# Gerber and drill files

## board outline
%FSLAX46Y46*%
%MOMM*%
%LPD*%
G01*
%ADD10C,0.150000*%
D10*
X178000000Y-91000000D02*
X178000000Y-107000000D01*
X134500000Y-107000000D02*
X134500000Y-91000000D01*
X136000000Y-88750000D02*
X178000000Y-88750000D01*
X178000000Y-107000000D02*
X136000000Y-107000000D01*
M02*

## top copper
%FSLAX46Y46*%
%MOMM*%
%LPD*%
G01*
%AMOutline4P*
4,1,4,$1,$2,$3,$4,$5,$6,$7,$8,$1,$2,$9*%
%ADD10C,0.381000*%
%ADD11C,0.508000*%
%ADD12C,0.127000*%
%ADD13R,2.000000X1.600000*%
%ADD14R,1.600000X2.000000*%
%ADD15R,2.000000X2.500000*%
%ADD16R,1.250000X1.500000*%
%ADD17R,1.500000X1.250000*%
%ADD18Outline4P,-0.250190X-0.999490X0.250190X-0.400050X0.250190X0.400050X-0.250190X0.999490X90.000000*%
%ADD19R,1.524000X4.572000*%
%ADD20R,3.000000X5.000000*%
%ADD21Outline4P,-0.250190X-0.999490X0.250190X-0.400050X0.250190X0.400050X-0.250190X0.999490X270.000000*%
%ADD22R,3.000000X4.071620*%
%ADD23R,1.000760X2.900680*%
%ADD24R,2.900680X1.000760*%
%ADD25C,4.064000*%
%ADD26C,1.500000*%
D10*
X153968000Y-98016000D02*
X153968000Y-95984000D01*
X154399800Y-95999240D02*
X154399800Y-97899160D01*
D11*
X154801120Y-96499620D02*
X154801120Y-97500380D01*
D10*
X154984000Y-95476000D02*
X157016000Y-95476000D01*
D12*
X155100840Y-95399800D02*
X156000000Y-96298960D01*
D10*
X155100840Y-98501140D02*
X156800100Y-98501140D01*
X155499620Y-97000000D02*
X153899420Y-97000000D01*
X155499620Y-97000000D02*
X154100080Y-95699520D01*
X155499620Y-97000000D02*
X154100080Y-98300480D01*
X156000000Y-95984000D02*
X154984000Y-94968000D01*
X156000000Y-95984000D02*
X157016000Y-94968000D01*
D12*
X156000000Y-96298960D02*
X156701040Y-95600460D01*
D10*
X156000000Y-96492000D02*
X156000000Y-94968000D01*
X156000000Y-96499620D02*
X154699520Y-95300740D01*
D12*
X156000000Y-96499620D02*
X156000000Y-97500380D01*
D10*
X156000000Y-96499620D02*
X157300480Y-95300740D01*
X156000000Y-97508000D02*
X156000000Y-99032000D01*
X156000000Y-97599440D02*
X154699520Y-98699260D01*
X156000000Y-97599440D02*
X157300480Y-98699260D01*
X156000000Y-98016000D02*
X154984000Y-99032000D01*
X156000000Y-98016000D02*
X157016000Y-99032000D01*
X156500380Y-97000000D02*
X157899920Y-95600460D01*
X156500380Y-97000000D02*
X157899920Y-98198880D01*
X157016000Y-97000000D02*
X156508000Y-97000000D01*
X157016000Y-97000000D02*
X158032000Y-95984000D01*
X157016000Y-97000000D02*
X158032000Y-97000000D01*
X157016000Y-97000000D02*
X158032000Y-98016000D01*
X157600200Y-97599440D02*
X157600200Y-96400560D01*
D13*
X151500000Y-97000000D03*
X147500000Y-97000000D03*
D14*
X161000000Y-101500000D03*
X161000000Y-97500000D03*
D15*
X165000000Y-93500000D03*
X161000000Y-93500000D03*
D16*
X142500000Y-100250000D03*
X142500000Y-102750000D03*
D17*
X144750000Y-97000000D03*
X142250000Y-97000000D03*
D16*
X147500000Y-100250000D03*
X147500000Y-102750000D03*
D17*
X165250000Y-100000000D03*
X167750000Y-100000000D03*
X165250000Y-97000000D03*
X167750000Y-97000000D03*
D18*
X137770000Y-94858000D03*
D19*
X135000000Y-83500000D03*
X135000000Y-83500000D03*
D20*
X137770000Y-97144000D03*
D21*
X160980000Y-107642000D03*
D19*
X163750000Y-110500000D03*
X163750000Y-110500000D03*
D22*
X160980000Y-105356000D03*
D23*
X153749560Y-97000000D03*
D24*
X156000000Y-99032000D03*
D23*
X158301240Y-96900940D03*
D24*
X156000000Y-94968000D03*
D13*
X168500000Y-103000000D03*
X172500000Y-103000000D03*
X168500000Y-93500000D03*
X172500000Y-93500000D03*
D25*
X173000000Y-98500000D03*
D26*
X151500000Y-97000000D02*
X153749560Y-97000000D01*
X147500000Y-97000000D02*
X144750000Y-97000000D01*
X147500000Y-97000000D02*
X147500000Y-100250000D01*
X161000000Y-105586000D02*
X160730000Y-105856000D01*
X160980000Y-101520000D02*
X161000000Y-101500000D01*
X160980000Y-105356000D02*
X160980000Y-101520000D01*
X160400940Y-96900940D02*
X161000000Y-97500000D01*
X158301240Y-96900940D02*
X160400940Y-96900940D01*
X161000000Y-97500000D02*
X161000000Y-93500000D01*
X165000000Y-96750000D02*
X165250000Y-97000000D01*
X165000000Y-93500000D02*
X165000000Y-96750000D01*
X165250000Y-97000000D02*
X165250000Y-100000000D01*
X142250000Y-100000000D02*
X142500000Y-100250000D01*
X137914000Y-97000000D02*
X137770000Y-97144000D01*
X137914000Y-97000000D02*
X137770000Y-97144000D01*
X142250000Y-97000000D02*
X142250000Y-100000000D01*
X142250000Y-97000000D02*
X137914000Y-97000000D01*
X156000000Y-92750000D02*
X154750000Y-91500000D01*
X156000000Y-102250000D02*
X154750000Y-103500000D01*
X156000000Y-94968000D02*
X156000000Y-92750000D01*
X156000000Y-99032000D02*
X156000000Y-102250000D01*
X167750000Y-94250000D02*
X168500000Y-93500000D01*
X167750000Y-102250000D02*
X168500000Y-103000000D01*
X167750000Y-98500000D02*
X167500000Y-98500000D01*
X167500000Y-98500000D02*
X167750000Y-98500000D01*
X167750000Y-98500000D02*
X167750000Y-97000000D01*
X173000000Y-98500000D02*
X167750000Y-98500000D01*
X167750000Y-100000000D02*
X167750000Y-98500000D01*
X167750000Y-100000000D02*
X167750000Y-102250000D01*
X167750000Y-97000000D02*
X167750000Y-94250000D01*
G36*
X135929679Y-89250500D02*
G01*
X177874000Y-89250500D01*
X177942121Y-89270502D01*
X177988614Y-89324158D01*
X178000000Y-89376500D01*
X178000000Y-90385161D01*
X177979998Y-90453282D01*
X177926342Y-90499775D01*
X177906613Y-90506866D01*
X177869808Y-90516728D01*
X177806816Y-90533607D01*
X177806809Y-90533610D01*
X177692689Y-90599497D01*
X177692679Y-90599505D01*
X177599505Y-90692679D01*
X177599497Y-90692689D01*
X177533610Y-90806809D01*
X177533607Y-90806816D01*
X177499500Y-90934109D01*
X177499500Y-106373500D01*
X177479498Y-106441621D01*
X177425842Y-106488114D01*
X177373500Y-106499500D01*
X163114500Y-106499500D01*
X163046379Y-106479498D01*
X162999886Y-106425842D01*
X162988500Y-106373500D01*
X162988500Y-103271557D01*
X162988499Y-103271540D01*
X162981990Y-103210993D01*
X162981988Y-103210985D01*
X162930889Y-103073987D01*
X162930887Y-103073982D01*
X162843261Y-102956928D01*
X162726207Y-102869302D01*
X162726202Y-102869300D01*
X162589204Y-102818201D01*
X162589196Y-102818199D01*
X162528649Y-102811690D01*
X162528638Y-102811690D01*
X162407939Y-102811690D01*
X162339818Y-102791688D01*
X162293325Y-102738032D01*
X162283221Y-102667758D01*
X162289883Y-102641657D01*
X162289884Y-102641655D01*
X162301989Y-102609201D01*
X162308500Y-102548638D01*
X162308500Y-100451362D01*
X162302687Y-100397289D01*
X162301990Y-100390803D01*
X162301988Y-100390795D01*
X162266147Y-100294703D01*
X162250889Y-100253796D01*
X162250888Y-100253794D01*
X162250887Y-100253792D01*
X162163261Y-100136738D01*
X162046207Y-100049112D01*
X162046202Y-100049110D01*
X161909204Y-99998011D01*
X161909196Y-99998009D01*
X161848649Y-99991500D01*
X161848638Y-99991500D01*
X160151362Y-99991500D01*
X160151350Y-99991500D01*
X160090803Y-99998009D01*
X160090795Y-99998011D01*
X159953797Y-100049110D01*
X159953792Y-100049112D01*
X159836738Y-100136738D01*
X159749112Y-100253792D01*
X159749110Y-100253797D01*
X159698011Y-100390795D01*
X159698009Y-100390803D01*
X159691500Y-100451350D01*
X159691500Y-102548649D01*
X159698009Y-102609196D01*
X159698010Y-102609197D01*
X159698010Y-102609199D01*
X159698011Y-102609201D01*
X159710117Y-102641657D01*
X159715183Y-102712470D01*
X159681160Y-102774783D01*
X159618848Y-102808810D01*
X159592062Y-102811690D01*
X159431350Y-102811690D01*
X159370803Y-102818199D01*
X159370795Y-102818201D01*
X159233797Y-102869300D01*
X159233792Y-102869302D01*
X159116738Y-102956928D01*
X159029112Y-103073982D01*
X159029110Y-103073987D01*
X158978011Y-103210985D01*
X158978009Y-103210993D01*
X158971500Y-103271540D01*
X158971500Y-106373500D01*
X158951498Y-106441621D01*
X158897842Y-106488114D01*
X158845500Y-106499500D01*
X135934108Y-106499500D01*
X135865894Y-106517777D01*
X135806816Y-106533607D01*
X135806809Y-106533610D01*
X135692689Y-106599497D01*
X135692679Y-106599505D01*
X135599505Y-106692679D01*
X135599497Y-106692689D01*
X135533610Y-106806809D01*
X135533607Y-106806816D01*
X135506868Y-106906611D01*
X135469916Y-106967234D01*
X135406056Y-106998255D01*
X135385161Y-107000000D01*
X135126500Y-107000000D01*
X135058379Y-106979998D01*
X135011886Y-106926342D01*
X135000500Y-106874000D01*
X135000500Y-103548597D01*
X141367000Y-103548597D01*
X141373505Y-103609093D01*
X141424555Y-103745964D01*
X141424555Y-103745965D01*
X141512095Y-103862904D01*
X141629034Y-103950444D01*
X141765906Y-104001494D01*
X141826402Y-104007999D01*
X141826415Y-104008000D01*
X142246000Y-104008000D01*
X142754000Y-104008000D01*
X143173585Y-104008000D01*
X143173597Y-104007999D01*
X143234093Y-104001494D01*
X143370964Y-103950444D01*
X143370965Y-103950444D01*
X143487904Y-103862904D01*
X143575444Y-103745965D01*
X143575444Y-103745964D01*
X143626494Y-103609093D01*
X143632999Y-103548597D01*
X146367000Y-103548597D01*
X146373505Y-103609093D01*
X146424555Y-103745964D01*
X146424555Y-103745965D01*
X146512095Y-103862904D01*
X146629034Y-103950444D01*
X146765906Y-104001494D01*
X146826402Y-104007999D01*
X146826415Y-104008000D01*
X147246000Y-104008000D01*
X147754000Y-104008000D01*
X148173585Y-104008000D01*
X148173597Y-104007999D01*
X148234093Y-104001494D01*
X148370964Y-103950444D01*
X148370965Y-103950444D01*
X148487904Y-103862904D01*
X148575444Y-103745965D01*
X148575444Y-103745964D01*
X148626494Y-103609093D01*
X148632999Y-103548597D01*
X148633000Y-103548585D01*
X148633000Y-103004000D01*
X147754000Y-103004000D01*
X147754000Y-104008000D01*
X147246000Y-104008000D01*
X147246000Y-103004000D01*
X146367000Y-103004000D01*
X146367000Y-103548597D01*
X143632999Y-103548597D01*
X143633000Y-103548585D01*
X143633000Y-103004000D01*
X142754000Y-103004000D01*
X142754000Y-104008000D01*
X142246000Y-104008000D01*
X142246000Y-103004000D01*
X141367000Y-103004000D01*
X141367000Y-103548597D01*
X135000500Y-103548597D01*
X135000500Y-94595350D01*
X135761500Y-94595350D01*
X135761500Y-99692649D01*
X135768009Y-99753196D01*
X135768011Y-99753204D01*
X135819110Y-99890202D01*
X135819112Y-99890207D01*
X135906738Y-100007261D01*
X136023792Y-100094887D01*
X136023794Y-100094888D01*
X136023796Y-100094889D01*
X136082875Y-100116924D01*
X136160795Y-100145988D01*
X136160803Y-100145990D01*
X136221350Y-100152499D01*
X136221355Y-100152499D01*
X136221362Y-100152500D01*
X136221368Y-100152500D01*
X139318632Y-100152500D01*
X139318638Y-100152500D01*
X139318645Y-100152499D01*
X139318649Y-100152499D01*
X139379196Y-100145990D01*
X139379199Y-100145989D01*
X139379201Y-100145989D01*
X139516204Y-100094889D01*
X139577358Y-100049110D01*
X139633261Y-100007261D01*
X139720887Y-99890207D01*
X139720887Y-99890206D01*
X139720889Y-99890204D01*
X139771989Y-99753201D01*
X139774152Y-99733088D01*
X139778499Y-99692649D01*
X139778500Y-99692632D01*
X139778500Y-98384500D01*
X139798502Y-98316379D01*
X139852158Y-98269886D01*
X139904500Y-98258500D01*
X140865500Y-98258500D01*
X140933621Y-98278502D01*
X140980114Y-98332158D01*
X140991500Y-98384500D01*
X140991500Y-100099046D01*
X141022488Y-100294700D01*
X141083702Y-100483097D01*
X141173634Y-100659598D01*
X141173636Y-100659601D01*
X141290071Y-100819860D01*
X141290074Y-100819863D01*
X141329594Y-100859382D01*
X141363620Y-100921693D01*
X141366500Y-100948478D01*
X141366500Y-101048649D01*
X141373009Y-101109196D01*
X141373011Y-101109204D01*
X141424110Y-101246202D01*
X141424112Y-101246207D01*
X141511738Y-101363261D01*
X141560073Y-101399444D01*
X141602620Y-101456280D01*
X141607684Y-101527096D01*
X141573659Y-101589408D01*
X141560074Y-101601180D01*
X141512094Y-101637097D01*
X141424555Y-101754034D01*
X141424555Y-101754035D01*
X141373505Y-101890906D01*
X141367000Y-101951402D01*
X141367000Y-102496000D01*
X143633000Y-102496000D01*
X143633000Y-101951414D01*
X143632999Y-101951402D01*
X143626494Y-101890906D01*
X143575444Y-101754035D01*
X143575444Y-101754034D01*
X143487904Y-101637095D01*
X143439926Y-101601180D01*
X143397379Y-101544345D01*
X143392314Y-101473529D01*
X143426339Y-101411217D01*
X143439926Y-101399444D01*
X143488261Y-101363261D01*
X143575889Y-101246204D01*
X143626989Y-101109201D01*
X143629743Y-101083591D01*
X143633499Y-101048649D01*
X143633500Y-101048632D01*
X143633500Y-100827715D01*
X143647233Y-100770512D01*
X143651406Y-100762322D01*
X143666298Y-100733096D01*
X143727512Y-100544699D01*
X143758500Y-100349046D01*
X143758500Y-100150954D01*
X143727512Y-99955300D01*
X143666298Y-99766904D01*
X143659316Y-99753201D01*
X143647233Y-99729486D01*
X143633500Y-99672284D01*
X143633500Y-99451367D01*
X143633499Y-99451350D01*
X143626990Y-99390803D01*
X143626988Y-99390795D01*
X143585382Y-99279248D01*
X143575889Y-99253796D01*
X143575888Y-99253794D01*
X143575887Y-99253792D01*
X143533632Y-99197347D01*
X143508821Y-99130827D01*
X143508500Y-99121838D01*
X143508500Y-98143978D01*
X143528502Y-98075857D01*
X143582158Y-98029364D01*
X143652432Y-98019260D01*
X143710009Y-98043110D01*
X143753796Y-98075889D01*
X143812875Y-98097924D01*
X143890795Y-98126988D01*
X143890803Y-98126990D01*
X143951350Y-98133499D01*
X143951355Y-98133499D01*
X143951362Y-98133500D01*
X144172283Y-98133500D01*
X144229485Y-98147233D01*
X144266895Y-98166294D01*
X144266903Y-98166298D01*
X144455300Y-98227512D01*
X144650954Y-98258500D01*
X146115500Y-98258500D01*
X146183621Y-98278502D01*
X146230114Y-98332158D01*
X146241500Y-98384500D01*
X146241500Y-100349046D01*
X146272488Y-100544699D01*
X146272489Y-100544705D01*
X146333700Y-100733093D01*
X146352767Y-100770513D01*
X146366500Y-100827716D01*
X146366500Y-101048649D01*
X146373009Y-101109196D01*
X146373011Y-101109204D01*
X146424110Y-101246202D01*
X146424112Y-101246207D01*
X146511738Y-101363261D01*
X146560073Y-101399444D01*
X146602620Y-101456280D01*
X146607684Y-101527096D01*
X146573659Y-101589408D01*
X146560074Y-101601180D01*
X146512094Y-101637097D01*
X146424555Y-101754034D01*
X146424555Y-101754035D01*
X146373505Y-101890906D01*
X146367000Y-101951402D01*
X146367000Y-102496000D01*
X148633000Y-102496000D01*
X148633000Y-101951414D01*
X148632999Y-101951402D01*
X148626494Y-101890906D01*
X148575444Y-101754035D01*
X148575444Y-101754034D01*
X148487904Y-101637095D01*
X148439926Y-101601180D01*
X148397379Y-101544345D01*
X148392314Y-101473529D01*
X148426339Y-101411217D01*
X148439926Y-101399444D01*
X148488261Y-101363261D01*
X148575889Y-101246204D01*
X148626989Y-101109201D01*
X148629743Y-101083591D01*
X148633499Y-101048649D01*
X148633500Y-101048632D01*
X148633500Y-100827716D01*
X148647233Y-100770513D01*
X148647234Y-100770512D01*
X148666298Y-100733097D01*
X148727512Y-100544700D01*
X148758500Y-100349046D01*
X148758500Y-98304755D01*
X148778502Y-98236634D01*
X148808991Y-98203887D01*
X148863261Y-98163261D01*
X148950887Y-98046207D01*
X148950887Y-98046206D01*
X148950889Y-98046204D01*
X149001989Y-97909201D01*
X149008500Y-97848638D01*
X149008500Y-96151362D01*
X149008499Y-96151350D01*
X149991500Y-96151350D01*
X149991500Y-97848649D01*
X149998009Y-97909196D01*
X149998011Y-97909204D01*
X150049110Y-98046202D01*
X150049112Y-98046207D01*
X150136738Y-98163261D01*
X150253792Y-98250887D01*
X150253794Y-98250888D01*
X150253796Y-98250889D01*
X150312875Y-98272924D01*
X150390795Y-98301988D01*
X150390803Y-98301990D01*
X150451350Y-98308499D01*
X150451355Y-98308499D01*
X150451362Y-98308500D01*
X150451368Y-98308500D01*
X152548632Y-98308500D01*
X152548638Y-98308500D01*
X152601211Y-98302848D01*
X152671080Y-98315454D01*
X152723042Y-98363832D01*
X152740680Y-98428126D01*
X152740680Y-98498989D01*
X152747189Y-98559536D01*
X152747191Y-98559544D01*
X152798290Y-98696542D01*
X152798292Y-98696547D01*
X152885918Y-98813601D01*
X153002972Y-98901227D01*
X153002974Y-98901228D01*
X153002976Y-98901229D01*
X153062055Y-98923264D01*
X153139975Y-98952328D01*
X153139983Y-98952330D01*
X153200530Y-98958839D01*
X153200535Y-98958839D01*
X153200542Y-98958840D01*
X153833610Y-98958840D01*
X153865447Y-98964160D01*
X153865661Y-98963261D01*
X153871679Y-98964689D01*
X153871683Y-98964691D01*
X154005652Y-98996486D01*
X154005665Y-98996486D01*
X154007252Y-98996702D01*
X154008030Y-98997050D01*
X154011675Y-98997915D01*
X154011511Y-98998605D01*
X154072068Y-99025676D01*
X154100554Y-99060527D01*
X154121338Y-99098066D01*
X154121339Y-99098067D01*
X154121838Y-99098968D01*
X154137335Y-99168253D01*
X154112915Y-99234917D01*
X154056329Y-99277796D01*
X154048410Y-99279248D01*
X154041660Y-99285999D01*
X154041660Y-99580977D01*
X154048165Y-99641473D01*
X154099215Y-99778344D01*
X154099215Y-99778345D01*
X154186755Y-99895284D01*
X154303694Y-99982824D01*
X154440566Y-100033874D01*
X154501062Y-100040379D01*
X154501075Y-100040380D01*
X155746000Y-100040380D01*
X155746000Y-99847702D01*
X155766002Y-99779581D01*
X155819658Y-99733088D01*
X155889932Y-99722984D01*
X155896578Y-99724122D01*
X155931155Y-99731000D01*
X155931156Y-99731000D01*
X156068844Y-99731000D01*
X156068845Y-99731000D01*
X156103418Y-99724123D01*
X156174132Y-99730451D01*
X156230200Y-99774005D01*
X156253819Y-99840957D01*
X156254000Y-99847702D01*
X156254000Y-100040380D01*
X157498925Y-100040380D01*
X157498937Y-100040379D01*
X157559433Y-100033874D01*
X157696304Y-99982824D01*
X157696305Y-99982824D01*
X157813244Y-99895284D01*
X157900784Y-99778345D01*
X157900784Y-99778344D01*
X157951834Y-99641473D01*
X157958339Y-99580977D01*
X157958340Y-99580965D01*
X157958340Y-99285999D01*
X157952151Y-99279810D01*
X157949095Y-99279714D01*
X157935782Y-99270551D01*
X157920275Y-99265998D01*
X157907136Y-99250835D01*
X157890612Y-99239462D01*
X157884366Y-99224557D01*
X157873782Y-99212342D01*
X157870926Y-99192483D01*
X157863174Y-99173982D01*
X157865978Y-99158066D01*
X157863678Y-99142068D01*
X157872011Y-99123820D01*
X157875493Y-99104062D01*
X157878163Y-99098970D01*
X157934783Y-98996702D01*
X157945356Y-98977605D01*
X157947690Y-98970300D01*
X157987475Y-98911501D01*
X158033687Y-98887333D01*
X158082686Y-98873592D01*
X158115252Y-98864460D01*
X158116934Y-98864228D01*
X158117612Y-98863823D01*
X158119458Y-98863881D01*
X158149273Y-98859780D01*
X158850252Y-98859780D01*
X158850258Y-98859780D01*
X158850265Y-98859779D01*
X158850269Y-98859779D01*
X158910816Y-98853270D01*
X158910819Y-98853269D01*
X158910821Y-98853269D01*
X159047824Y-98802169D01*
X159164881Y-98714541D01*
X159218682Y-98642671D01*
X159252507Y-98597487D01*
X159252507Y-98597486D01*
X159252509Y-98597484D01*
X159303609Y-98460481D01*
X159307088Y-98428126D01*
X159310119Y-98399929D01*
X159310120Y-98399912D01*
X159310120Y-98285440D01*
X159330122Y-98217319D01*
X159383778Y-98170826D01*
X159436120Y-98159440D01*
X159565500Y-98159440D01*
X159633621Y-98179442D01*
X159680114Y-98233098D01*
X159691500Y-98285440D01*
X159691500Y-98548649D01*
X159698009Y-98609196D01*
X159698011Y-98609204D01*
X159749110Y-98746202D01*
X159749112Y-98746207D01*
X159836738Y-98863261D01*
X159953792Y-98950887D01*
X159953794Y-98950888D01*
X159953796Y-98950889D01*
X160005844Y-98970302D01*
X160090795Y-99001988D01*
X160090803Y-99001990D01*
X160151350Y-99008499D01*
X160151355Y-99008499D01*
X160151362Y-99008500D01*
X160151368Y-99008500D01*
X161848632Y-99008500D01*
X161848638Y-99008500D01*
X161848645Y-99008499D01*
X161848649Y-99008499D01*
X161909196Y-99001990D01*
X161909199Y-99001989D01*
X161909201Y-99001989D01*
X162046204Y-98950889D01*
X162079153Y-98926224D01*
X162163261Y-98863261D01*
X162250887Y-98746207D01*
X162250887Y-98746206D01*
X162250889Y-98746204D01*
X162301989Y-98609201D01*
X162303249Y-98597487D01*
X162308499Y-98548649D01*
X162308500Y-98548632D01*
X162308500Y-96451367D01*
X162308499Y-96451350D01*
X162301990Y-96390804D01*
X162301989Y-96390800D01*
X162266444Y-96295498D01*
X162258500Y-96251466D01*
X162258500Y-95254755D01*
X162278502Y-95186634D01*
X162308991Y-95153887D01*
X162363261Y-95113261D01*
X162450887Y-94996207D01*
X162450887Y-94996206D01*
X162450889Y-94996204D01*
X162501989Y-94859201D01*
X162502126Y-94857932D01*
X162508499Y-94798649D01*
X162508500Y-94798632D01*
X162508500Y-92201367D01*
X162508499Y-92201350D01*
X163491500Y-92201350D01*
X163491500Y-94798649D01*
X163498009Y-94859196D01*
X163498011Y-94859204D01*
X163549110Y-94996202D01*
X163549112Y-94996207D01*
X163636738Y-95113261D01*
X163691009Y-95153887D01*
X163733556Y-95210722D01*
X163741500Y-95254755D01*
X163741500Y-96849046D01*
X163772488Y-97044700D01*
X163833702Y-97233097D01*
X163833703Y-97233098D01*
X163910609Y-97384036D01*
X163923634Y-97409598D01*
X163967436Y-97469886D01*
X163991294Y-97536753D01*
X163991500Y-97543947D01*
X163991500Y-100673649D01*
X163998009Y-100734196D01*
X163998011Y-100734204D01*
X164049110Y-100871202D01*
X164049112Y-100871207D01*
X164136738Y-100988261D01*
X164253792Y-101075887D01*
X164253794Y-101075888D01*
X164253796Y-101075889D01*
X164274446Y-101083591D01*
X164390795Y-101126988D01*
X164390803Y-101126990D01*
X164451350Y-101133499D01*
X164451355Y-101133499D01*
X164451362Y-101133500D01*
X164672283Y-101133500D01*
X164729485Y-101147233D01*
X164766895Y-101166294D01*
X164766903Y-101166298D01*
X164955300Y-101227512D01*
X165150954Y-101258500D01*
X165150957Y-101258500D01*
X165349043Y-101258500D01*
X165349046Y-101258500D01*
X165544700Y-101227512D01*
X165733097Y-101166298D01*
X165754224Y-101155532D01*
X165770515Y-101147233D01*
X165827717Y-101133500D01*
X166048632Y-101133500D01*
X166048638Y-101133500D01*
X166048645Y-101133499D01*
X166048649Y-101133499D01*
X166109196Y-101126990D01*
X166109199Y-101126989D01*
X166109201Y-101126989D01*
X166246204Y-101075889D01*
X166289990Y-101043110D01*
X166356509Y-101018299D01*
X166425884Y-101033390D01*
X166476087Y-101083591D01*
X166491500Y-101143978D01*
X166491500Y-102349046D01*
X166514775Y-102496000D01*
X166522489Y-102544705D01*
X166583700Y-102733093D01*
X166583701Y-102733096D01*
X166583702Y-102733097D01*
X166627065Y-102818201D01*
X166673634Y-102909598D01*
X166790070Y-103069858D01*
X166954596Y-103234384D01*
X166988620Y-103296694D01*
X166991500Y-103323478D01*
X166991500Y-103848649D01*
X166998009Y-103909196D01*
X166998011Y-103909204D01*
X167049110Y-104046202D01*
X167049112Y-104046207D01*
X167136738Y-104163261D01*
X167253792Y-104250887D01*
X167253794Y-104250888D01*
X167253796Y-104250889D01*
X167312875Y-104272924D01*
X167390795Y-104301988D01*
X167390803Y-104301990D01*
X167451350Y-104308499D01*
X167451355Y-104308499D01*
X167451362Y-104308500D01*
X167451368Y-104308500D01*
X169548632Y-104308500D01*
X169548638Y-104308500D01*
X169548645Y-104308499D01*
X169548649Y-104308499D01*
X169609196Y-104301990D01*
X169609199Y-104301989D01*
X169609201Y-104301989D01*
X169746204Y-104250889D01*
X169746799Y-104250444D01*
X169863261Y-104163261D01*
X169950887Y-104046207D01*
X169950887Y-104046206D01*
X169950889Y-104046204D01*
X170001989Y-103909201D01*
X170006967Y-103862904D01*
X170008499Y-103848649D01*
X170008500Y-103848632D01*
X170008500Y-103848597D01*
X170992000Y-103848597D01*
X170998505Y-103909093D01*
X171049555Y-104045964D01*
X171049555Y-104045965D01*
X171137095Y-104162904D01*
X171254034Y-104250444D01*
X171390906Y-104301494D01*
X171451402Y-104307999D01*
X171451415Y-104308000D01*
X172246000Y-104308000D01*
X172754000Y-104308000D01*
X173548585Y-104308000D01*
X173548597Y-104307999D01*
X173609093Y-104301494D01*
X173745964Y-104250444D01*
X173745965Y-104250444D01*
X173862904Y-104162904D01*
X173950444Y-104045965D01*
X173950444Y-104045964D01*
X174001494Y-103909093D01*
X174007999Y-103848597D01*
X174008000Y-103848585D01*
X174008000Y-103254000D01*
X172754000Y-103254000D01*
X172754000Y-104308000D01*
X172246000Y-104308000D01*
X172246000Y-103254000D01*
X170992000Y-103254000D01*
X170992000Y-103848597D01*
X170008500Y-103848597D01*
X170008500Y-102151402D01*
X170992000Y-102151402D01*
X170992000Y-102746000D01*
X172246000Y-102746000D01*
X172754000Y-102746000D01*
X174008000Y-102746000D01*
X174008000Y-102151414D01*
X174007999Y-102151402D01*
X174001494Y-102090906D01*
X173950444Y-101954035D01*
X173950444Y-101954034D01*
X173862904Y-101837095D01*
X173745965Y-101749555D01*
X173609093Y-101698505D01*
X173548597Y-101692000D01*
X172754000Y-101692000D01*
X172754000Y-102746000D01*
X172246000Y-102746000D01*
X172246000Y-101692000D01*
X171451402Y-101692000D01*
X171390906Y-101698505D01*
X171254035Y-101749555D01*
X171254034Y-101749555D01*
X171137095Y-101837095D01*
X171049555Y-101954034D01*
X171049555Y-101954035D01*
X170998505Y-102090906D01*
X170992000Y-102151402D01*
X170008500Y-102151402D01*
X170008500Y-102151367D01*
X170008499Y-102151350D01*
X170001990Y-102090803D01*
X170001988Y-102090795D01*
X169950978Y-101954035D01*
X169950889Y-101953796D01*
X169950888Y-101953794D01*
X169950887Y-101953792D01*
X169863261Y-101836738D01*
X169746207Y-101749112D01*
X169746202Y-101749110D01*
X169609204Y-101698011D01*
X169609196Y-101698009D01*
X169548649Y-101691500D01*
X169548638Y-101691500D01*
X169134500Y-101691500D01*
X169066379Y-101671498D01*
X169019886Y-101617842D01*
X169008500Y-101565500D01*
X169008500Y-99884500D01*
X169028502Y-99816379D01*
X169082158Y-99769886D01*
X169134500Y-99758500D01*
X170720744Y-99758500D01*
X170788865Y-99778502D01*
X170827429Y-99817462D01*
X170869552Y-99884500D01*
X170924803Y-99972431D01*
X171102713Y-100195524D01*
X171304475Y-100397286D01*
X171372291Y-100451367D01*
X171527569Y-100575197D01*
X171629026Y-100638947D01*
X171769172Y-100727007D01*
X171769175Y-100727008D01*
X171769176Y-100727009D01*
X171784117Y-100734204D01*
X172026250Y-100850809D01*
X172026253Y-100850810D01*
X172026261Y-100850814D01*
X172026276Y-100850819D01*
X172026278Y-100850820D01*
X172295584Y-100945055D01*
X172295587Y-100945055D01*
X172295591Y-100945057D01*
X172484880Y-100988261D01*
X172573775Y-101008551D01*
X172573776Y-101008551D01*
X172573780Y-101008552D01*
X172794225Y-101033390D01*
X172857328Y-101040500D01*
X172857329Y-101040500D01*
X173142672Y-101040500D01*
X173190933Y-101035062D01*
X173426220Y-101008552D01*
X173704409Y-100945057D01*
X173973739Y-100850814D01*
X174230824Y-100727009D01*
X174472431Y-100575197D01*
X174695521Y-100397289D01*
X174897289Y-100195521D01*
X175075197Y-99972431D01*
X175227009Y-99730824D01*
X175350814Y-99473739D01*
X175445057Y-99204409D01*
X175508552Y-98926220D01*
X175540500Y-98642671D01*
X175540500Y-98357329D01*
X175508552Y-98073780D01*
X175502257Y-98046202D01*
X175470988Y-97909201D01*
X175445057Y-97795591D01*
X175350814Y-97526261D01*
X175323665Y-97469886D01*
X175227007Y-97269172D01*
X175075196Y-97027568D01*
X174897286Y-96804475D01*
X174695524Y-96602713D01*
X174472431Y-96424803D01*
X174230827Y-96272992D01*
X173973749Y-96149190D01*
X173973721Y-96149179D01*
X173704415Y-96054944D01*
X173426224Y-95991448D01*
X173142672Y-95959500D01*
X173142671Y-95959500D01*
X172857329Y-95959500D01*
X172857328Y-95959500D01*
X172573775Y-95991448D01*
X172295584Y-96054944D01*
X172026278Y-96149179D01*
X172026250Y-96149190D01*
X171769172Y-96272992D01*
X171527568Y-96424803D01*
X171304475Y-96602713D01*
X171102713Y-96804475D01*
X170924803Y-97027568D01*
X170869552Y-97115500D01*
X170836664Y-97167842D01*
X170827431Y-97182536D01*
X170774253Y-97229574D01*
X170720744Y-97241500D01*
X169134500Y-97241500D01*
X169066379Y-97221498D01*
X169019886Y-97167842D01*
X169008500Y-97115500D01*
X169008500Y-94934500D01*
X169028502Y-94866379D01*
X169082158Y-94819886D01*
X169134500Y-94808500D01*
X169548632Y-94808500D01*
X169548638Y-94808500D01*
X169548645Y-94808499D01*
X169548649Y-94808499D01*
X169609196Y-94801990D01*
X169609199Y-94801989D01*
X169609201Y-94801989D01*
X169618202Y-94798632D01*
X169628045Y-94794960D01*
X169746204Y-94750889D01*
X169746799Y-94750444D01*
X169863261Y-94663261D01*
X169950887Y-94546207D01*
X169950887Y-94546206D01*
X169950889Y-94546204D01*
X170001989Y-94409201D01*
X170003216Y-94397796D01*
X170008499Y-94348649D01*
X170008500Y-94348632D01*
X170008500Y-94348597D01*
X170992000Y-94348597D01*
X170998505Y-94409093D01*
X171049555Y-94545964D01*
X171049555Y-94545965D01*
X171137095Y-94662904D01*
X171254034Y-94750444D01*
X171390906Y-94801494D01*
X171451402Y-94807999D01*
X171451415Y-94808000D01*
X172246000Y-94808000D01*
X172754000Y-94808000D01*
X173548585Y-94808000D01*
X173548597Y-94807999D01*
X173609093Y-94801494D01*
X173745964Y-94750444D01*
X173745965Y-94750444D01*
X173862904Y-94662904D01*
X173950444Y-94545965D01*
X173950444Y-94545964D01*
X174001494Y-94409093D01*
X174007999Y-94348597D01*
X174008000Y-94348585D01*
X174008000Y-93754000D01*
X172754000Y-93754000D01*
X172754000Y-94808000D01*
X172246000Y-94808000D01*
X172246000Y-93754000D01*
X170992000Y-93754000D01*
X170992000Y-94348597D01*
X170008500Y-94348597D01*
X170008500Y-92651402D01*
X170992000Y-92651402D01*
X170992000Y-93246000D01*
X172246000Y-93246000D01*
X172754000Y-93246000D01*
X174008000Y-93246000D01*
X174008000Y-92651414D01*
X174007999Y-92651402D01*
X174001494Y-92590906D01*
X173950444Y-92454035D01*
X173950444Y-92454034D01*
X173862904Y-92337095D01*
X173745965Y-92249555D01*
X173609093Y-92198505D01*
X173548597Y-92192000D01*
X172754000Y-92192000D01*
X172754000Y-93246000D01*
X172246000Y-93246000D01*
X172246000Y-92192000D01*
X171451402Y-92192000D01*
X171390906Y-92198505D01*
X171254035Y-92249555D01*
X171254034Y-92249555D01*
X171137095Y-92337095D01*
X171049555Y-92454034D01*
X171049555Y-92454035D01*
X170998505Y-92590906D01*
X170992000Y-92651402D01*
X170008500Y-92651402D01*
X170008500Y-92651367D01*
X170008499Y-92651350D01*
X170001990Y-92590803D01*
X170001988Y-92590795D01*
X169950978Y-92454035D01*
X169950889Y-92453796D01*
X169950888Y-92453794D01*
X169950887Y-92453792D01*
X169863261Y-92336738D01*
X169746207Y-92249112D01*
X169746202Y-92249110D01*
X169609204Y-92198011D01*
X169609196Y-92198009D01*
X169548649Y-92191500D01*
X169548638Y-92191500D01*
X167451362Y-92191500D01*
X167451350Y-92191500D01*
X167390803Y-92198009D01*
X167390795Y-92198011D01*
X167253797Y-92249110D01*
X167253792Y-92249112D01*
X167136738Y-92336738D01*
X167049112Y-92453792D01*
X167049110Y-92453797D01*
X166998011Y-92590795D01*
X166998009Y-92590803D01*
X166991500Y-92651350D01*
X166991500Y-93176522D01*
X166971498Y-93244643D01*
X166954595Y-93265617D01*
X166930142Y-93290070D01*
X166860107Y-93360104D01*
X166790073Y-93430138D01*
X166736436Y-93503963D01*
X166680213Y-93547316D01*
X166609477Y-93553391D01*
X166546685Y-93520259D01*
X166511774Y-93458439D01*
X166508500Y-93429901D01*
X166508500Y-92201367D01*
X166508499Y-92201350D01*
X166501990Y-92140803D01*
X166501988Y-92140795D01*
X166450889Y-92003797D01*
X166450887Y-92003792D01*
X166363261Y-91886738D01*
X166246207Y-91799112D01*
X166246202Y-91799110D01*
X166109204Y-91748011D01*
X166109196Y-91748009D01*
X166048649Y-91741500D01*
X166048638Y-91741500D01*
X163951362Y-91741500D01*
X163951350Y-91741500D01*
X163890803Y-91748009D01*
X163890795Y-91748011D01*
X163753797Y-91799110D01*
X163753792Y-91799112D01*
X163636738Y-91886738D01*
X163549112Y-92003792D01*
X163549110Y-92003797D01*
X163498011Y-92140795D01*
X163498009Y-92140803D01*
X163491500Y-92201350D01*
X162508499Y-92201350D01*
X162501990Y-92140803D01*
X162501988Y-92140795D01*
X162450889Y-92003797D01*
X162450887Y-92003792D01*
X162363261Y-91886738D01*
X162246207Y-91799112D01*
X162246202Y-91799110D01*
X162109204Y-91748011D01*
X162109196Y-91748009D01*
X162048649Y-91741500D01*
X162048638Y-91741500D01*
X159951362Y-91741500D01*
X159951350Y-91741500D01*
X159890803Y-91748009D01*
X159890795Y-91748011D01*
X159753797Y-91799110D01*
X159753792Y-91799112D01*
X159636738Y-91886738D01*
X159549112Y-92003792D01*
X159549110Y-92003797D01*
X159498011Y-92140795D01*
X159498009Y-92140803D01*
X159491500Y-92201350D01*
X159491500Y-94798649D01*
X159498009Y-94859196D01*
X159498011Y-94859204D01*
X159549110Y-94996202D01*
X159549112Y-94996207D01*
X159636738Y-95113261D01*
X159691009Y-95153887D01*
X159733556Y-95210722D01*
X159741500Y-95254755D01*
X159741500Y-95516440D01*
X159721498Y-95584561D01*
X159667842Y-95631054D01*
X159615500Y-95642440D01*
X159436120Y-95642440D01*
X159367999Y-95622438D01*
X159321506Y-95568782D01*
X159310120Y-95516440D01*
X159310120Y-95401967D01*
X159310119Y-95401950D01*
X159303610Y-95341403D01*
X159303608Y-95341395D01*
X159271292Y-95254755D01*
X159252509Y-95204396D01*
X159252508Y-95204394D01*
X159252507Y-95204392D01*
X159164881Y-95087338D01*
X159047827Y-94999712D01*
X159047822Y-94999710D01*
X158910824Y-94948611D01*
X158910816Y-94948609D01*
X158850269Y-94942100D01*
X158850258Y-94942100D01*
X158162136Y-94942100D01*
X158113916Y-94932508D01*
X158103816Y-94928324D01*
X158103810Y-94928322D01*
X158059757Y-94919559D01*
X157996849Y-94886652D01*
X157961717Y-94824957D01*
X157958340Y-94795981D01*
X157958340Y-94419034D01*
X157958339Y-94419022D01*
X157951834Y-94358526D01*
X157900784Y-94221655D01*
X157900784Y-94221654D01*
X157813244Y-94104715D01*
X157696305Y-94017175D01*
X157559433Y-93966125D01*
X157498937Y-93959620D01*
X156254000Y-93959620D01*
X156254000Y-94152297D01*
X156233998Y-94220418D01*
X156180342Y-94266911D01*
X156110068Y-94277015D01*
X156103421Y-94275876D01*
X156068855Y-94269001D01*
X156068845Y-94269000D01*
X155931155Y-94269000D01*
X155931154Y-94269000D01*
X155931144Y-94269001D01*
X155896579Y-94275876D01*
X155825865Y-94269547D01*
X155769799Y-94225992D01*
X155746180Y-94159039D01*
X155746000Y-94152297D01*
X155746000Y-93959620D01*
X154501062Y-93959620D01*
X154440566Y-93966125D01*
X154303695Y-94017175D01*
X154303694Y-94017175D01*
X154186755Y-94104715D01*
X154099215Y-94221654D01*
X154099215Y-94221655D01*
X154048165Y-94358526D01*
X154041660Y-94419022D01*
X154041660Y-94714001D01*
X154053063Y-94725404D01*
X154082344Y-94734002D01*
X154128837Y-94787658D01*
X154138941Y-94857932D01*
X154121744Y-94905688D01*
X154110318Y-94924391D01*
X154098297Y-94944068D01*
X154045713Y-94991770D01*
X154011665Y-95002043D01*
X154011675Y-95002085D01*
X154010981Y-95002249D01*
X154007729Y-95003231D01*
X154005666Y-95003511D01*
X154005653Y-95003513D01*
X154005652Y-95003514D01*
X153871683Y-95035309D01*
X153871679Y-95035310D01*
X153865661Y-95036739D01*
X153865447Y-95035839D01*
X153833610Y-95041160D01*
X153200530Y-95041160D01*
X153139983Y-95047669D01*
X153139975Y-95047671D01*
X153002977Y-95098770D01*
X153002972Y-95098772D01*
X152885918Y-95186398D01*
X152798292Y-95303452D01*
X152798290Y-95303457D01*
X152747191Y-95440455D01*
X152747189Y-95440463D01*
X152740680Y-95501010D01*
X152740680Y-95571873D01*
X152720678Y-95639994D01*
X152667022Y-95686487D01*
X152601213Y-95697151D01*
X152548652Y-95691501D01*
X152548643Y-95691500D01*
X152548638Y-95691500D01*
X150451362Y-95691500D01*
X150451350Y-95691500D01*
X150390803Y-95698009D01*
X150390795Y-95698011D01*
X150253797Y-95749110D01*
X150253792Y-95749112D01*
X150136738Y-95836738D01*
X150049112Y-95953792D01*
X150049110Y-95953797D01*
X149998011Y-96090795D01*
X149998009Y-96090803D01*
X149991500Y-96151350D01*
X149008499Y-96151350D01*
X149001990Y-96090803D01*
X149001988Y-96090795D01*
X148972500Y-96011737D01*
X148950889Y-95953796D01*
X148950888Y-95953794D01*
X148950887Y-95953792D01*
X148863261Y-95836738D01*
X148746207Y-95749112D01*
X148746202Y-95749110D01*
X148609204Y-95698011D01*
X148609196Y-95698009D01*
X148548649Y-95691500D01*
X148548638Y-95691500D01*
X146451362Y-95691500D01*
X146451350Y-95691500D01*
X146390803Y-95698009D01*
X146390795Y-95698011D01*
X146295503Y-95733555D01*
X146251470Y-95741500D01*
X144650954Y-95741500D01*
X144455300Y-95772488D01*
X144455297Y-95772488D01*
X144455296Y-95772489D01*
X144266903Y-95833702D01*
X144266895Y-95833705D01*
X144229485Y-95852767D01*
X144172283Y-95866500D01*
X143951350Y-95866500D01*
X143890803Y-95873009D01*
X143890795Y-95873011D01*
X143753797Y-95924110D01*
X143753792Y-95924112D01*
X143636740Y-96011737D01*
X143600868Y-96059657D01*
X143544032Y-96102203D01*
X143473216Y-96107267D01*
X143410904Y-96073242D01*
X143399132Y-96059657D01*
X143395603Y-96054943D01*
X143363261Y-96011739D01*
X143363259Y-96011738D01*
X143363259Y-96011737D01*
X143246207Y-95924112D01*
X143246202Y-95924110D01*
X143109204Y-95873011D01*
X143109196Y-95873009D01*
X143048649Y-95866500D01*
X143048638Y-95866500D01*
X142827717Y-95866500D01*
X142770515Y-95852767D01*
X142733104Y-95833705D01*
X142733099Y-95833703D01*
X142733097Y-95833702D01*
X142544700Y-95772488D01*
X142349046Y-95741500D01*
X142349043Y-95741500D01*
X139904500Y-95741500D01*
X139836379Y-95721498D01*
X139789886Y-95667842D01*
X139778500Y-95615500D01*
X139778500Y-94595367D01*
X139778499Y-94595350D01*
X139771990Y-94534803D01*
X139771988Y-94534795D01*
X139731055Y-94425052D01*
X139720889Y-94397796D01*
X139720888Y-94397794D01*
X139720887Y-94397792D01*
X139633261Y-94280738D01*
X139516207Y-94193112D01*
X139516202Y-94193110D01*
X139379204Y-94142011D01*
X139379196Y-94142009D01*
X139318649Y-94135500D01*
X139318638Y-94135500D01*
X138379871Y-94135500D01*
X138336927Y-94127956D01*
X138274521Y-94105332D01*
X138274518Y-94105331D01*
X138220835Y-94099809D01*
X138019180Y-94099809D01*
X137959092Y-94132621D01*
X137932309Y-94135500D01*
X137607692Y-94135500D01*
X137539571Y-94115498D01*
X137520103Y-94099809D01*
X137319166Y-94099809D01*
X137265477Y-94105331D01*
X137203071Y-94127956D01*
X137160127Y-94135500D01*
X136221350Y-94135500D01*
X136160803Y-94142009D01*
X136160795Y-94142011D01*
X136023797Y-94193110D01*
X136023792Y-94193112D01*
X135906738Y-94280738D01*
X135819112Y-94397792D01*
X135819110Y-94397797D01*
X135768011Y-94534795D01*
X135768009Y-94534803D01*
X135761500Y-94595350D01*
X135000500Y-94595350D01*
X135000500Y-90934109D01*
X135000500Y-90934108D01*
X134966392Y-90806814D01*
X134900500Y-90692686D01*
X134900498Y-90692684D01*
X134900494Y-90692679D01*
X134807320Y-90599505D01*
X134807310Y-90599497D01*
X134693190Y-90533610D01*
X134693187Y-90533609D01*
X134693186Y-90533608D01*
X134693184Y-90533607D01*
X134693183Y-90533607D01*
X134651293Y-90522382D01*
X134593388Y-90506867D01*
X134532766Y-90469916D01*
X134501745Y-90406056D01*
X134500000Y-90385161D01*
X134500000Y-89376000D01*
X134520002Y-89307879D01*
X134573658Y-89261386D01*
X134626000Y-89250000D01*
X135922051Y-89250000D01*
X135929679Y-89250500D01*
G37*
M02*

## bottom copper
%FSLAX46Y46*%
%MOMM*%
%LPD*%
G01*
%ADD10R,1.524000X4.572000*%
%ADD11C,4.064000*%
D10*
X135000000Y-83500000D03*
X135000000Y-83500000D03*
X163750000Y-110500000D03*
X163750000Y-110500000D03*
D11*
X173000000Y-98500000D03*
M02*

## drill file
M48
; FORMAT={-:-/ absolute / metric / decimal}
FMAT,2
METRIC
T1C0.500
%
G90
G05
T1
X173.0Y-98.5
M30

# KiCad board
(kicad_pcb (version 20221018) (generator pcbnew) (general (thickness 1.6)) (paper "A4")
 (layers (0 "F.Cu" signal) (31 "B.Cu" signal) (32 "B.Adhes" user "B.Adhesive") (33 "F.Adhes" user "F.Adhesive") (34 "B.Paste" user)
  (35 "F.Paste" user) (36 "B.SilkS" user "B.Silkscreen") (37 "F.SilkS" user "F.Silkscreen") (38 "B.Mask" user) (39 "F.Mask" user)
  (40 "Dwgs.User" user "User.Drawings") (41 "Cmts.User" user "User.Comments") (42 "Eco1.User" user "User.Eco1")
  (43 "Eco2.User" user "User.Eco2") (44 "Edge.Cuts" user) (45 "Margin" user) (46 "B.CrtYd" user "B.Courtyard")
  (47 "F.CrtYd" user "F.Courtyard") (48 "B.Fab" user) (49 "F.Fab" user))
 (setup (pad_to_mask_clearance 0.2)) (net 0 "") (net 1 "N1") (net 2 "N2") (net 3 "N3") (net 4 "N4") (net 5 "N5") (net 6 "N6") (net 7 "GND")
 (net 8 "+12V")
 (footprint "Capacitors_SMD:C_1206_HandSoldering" (layer "F.Cu") (at 149.5 97 180)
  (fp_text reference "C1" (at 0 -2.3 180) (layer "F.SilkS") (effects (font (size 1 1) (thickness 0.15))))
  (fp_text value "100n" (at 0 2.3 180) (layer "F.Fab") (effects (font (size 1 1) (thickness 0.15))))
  (pad "1" smd rect (at -2 0 180) (size 2 1.6) (layers "F.Cu" "F.Paste" "F.Mask") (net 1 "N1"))
  (pad "2" smd rect (at 2 0 180) (size 2 1.6) (layers "F.Cu" "F.Paste" "F.Mask") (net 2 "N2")))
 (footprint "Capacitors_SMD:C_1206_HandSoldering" (layer "F.Cu") (at 161 99.5 90)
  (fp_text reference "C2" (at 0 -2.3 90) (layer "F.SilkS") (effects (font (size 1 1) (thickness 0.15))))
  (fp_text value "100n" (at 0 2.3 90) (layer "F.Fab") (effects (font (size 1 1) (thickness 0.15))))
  (pad "1" smd rect (at -2 0 90) (size 2 1.6) (layers "F.Cu" "F.Paste" "F.Mask") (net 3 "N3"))
  (pad "2" smd rect (at 2 0 90) (size 2 1.6) (layers "F.Cu" "F.Paste" "F.Mask") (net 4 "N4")))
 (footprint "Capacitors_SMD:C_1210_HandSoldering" (layer "F.Cu") (at 163 93.5 180)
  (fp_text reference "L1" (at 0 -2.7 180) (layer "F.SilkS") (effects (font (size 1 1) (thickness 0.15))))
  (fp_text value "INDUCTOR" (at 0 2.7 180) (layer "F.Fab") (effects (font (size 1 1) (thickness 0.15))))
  (pad "1" smd rect (at -2 0 180) (size 2 2.5) (layers "F.Cu" "F.Paste" "F.Mask") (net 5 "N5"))
  (pad "2" smd rect (at 2 0 180) (size 2 2.5) (layers "F.Cu" "F.Paste" "F.Mask") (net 4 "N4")))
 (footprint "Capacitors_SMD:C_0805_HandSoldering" (layer "F.Cu") (at 142.5 101.5 -90)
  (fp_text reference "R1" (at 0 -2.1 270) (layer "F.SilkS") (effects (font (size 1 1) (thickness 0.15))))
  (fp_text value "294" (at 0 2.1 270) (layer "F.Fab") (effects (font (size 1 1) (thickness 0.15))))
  (pad "1" smd rect (at -1.25 0 270) (size 1.5 1.25) (layers "F.Cu" "F.Paste" "F.Mask") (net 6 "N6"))
  (pad "2" smd rect (at 1.25 0 270) (size 1.5 1.25) (layers "F.Cu" "F.Paste" "F.Mask") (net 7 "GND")))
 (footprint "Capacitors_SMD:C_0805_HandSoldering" (layer "F.Cu") (at 143.5 97 180)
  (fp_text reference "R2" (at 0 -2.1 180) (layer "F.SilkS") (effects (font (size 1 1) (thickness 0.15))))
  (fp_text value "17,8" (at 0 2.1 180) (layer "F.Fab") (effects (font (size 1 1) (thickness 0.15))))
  (pad "1" smd rect (at -1.25 0 180) (size 1.5 1.25) (layers "F.Cu" "F.Paste" "F.Mask") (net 2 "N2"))
  (pad "2" smd rect (at 1.25 0 180) (size 1.5 1.25) (layers "F.Cu" "F.Paste" "F.Mask") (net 6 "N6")))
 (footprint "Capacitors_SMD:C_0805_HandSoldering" (layer "F.Cu") (at 147.5 101.5 -90)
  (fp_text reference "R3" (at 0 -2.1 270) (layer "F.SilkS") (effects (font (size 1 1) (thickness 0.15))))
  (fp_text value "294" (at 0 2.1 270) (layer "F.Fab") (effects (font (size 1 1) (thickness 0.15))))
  (pad "1" smd rect (at -1.25 0 270) (size 1.5 1.25) (layers "F.Cu" "F.Paste" "F.Mask") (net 2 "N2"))
  (pad "2" smd rect (at 1.25 0 270) (size 1.5 1.25) (layers "F.Cu" "F.Paste" "F.Mask") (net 7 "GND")))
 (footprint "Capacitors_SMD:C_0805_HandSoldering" (layer "F.Cu") (at 166.5 100)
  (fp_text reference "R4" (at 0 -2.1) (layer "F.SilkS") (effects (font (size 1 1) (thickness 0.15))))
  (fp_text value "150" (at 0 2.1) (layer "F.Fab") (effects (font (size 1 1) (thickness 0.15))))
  (pad "1" smd rect (at -1.25 0) (size 1.5 1.25) (layers "F.Cu" "F.Paste" "F.Mask") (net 5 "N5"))
  (pad "2" smd rect (at 1.25 0) (size 1.5 1.25) (layers "F.Cu" "F.Paste" "F.Mask") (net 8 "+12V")))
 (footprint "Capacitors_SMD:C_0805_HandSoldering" (layer "F.Cu") (at 166.5 97)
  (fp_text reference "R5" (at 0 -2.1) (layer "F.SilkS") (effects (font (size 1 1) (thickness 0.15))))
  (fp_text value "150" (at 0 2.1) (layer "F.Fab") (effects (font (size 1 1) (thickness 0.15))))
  (pad "1" smd rect (at -1.25 0) (size 1.5 1.25) (layers "F.Cu" "F.Paste" "F.Mask") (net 5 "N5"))
  (pad "2" smd rect (at 1.25 0) (size 1.5 1.25) (layers "F.Cu" "F.Paste" "F.Mask") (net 8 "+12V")))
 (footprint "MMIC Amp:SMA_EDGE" (layer "F.Cu") (at 136.5 88 90)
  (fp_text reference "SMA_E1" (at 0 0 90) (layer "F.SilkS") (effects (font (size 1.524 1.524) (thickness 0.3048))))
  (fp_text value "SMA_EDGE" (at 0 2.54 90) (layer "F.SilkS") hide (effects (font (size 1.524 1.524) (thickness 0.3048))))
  (pad "1" connect trapezoid (at -6.858 1.27 90) (size 0.50038 1.39954) (rect_delta 0.59944 0) (layers "F.Cu" "F.Mask") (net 7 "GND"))
  (pad "1" connect rect (at 4.5 -1.5 90) (size 4.572 1.524) (layers "*.Cu" "F.Mask") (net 7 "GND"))
  (pad "2" connect rect (at 4.5 -1.5 90) (size 4.572 1.524) (layers "*.Cu" "F.Mask") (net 7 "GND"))
  (pad "3" connect rect (at -9.144 1.27 90) (size 5 3) (layers "F.Cu" "F.Mask") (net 6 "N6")))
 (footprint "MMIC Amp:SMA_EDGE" (layer "F.Cu") (at 162.25 114.5 -90)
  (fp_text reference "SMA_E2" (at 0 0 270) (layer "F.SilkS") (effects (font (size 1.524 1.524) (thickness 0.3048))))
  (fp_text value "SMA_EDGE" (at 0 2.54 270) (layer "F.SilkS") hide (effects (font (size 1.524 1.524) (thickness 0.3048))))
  (pad "1" connect trapezoid (at -6.858 1.27 270) (size 0.50038 1.39954) (rect_delta 0.59944 0) (layers "F.Cu" "F.Mask") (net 7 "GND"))
  (pad "1" connect rect (at -4 -1.5 270) (size 4.572 1.524) (layers "*.Cu" "F.Mask") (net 7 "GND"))
  (pad "2" connect rect (at -4 -1.5 270) (size 4.572 1.524) (layers "*.Cu" "F.Mask") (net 7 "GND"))
  (pad "3" connect rect (at -9.144 1.27 270) (size 4.07162 3) (layers "F.Cu" "F.Mask") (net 3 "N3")))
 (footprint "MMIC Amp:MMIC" (layer "F.Cu") (at 156 97)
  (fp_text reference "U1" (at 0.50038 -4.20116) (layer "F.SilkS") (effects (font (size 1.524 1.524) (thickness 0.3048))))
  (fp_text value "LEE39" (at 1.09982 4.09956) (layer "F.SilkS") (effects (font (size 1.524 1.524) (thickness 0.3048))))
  (fp_line (start -2.032 1.016) (end -2.032 -1.016) (stroke (width 0.381) (type solid)) (layer "F.Cu"))
  (fp_line (start -1.6002 -1.00076) (end -1.6002 0.89916) (stroke (width 0.381) (type solid)) (layer "F.Cu"))
  (fp_line (start -1.19888 -0.50038) (end -1.19888 0.50038) (stroke (width 0.508) (type solid)) (layer "F.Cu"))
  (fp_line (start -1.016 -1.524) (end 1.016 -1.524) (stroke (width 0.381) (type solid)) (layer "F.Cu"))
  (fp_line (start -0.89916 -1.6002) (end 0 -0.70104) (stroke (width 0.127) (type solid)) (layer "F.Cu"))
  (fp_line (start -0.89916 1.50114) (end 0.8001 1.50114) (stroke (width 0.381) (type solid)) (layer "F.Cu"))
  (fp_line (start -0.50038 0) (end -2.10058 0) (stroke (width 0.381) (type solid)) (layer "F.Cu"))
  (fp_line (start -0.50038 0) (end -1.89992 -1.30048) (stroke (width 0.381) (type solid)) (layer "F.Cu"))
  (fp_line (start -0.50038 0) (end -1.89992 1.30048) (stroke (width 0.381) (type solid)) (layer "F.Cu"))
  (fp_line (start 0 -1.016) (end -1.016 -2.032) (stroke (width 0.381) (type solid)) (layer "F.Cu"))
  (fp_line (start 0 -1.016) (end 1.016 -2.032) (stroke (width 0.381) (type solid)) (layer "F.Cu"))
  (fp_line (start 0 -0.70104) (end 0.70104 -1.39954) (stroke (width 0.127) (type solid)) (layer "F.Cu"))
  (fp_line (start 0 -0.508) (end 0 -2.032) (stroke (width 0.381) (type solid)) (layer "F.Cu"))
  (fp_line (start 0 -0.50038) (end -1.30048 -1.69926) (stroke (width 0.381) (type solid)) (layer "F.Cu"))
  (fp_line (start 0 -0.50038) (end 0 0.50038) (stroke (width 0.127) (type solid)) (layer "F.Cu"))
  (fp_line (start 0 -0.50038) (end 1.30048 -1.69926) (stroke (width 0.381) (type solid)) (layer "F.Cu"))
  (fp_line (start 0 0.508) (end 0 2.032) (stroke (width 0.381) (type solid)) (layer "F.Cu"))
  (fp_line (start 0 0.59944) (end -1.30048 1.69926) (stroke (width 0.381) (type solid)) (layer "F.Cu"))
  (fp_line (start 0 0.59944) (end 1.30048 1.69926) (stroke (width 0.381) (type solid)) (layer "F.Cu"))
  (fp_line (start 0 1.016) (end -1.016 2.032) (stroke (width 0.381) (type solid)) (layer "F.Cu"))
  (fp_line (start 0 1.016) (end 1.016 2.032) (stroke (width 0.381) (type solid)) (layer "F.Cu"))
  (fp_line (start 0.50038 0) (end 1.89992 -1.39954) (stroke (width 0.381) (type solid)) (layer "F.Cu"))
  (fp_line (start 0.50038 0) (end 1.89992 1.19888) (stroke (width 0.381) (type solid)) (layer "F.Cu"))
  (fp_line (start 1.016 0) (end 0.508 0) (stroke (width 0.381) (type solid)) (layer "F.Cu"))
  (fp_line (start 1.016 0) (end 2.032 -1.016) (stroke (width 0.381) (type solid)) (layer "F.Cu"))
  (fp_line (start 1.016 0) (end 2.032 0) (stroke (width 0.381) (type solid)) (layer "F.Cu"))
  (fp_line (start 1.016 0) (end 2.032 1.016) (stroke (width 0.381) (type solid)) (layer "F.Cu"))
  (fp_line (start 1.6002 0.59944) (end 1.6002 -0.59944) (stroke (width 0.381) (type solid)) (layer "F.Cu"))
  (pad "1" smd rect (at -2.25044 0) (size 1.00076 2.90068) (layers "F.Cu" "F.Paste" "F.Mask") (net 1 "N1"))
  (pad "2" smd rect (at 0 2.032) (size 2.90068 1.00076) (layers "F.Cu" "F.Paste" "F.Mask") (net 7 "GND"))
  (pad "3" smd rect (at 2.30124 -0.09906) (size 1.00076 2.90068) (layers "F.Cu" "F.Paste" "F.Mask") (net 4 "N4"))
  (pad "4" smd rect (at 0 -2.032) (size 2.90068 1.00076) (layers "F.Cu" "F.Paste" "F.Mask") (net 7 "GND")))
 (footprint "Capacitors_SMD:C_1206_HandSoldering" (layer "F.Cu") (at 170.5 103)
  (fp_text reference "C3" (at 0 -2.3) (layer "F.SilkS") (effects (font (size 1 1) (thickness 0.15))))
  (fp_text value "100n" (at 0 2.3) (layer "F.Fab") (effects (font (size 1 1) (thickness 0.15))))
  (pad "1" smd rect (at -2 0) (size 2 1.6) (layers "F.Cu" "F.Paste" "F.Mask") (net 8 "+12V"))
  (pad "2" smd rect (at 2 0) (size 2 1.6) (layers "F.Cu" "F.Paste" "F.Mask") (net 7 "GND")))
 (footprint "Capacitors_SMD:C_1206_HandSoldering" (layer "F.Cu") (at 170.5 93.5)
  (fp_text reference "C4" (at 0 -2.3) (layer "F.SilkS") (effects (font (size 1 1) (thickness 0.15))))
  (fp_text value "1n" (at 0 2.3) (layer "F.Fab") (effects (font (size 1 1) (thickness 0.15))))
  (pad "1" smd rect (at -2 0) (size 2 1.6) (layers "F.Cu" "F.Paste" "F.Mask") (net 8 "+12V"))
  (pad "2" smd rect (at 2 0) (size 2 1.6) (layers "F.Cu" "F.Paste" "F.Mask") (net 7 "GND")))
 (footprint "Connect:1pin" (layer "F.Cu") (at 173 98.5)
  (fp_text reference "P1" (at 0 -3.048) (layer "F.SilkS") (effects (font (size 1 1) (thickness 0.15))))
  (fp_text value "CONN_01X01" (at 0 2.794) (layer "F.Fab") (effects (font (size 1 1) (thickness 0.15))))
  (pad "1" thru_hole circle (at 0 0) (size 4.064 4.064) (drill 0.5) (layers "*.Cu" "*.Mask" "F.SilkS") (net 8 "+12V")))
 (gr_line (start 178 91) (end 178 107) (stroke (width 0.15) (type solid)) (layer "Edge.Cuts"))
 (gr_line (start 134.5 107) (end 134.5 91) (stroke (width 0.15) (type solid)) (layer "Edge.Cuts"))
 (gr_line (start 136 88.75) (end 178 88.75) (stroke (width 0.15) (type solid)) (layer "Edge.Cuts"))
 (gr_line (start 178 107) (end 136 107) (stroke (width 0.15) (type solid)) (layer "Edge.Cuts"))
 (segment (start 151.5 97) (end 153.74956 97) (width 1.5) (layer "F.Cu") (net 1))
 (segment (start 147.5 97) (end 144.75 97) (width 1.5) (layer "F.Cu") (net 2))
 (segment (start 147.5 97) (end 147.5 100.25) (width 1.5) (layer "F.Cu") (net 2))
 (segment (start 161 105.586) (end 160.73 105.856) (width 1.5) (layer "F.Cu") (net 3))
 (segment (start 160.98 101.52) (end 161 101.5) (width 1.5) (layer "F.Cu") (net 3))
 (segment (start 160.98 105.356) (end 160.98 101.52) (width 1.5) (layer "F.Cu") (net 3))
 (segment (start 160.40094 96.90094) (end 161 97.5) (width 1.5) (layer "F.Cu") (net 4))
 (segment (start 158.30124 96.90094) (end 160.40094 96.90094) (width 1.5) (layer "F.Cu") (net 4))
 (segment (start 161 97.5) (end 161 93.5) (width 1.5) (layer "F.Cu") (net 4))
 (segment (start 165 96.75) (end 165.25 97) (width 1.5) (layer "F.Cu") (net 5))
 (segment (start 165 93.5) (end 165 96.75) (width 1.5) (layer "F.Cu") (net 5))
 (segment (start 165.25 97) (end 165.25 100) (width 1.5) (layer "F.Cu") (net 5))
 (segment (start 142.25 100) (end 142.5 100.25) (width 1.5) (layer "F.Cu") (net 6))
 (segment (start 137.914 97) (end 137.77 97.144) (width 1.5) (layer "F.Cu") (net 6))
 (segment (start 137.914 97) (end 137.77 97.144) (width 1.5) (layer "F.Cu") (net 6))
 (segment (start 142.25 97) (end 142.25 100) (width 1.5) (layer "F.Cu") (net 6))
 (segment (start 142.25 97) (end 137.914 97) (width 1.5) (layer "F.Cu") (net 6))
 (segment (start 156 92.75) (end 154.75 91.5) (width 1.5) (layer "F.Cu") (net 7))
 (segment (start 156 102.25) (end 154.75 103.5) (width 1.5) (layer "F.Cu") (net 7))
 (segment (start 156 94.968) (end 156 92.75) (width 1.5) (layer "F.Cu") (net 7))
 (segment (start 156 99.032) (end 156 102.25) (width 1.5) (layer "F.Cu") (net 7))
 (segment (start 167.75 94.25) (end 168.5 93.5) (width 1.5) (layer "F.Cu") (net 8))
 (segment (start 167.75 102.25) (end 168.5 103) (width 1.5) (layer "F.Cu") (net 8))
 (segment (start 167.75 98.5) (end 167.5 98.5) (width 1.5) (layer "F.Cu") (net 8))
 (segment (start 167.5 98.5) (end 167.75 98.5) (width 1.5) (layer "F.Cu") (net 8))
 (segment (start 167.75 98.5) (end 167.75 97) (width 1.5) (layer "F.Cu") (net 8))
 (segment (start 173 98.5) (end 167.75 98.5) (width 1.5) (layer "F.Cu") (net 8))
 (segment (start 167.75 100) (end 167.75 98.5) (width 1.5) (layer "F.Cu") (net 8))
 (segment (start 167.75 100) (end 167.75 102.25) (width 1.5) (layer "F.Cu") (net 8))
 (segment (start 167.75 97) (end 167.75 94.25) (width 1.5) (layer "F.Cu") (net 8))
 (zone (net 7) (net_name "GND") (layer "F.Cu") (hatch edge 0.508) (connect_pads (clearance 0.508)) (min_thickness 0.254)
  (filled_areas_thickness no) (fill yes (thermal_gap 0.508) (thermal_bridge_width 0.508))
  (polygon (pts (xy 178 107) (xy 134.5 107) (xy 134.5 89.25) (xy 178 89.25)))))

